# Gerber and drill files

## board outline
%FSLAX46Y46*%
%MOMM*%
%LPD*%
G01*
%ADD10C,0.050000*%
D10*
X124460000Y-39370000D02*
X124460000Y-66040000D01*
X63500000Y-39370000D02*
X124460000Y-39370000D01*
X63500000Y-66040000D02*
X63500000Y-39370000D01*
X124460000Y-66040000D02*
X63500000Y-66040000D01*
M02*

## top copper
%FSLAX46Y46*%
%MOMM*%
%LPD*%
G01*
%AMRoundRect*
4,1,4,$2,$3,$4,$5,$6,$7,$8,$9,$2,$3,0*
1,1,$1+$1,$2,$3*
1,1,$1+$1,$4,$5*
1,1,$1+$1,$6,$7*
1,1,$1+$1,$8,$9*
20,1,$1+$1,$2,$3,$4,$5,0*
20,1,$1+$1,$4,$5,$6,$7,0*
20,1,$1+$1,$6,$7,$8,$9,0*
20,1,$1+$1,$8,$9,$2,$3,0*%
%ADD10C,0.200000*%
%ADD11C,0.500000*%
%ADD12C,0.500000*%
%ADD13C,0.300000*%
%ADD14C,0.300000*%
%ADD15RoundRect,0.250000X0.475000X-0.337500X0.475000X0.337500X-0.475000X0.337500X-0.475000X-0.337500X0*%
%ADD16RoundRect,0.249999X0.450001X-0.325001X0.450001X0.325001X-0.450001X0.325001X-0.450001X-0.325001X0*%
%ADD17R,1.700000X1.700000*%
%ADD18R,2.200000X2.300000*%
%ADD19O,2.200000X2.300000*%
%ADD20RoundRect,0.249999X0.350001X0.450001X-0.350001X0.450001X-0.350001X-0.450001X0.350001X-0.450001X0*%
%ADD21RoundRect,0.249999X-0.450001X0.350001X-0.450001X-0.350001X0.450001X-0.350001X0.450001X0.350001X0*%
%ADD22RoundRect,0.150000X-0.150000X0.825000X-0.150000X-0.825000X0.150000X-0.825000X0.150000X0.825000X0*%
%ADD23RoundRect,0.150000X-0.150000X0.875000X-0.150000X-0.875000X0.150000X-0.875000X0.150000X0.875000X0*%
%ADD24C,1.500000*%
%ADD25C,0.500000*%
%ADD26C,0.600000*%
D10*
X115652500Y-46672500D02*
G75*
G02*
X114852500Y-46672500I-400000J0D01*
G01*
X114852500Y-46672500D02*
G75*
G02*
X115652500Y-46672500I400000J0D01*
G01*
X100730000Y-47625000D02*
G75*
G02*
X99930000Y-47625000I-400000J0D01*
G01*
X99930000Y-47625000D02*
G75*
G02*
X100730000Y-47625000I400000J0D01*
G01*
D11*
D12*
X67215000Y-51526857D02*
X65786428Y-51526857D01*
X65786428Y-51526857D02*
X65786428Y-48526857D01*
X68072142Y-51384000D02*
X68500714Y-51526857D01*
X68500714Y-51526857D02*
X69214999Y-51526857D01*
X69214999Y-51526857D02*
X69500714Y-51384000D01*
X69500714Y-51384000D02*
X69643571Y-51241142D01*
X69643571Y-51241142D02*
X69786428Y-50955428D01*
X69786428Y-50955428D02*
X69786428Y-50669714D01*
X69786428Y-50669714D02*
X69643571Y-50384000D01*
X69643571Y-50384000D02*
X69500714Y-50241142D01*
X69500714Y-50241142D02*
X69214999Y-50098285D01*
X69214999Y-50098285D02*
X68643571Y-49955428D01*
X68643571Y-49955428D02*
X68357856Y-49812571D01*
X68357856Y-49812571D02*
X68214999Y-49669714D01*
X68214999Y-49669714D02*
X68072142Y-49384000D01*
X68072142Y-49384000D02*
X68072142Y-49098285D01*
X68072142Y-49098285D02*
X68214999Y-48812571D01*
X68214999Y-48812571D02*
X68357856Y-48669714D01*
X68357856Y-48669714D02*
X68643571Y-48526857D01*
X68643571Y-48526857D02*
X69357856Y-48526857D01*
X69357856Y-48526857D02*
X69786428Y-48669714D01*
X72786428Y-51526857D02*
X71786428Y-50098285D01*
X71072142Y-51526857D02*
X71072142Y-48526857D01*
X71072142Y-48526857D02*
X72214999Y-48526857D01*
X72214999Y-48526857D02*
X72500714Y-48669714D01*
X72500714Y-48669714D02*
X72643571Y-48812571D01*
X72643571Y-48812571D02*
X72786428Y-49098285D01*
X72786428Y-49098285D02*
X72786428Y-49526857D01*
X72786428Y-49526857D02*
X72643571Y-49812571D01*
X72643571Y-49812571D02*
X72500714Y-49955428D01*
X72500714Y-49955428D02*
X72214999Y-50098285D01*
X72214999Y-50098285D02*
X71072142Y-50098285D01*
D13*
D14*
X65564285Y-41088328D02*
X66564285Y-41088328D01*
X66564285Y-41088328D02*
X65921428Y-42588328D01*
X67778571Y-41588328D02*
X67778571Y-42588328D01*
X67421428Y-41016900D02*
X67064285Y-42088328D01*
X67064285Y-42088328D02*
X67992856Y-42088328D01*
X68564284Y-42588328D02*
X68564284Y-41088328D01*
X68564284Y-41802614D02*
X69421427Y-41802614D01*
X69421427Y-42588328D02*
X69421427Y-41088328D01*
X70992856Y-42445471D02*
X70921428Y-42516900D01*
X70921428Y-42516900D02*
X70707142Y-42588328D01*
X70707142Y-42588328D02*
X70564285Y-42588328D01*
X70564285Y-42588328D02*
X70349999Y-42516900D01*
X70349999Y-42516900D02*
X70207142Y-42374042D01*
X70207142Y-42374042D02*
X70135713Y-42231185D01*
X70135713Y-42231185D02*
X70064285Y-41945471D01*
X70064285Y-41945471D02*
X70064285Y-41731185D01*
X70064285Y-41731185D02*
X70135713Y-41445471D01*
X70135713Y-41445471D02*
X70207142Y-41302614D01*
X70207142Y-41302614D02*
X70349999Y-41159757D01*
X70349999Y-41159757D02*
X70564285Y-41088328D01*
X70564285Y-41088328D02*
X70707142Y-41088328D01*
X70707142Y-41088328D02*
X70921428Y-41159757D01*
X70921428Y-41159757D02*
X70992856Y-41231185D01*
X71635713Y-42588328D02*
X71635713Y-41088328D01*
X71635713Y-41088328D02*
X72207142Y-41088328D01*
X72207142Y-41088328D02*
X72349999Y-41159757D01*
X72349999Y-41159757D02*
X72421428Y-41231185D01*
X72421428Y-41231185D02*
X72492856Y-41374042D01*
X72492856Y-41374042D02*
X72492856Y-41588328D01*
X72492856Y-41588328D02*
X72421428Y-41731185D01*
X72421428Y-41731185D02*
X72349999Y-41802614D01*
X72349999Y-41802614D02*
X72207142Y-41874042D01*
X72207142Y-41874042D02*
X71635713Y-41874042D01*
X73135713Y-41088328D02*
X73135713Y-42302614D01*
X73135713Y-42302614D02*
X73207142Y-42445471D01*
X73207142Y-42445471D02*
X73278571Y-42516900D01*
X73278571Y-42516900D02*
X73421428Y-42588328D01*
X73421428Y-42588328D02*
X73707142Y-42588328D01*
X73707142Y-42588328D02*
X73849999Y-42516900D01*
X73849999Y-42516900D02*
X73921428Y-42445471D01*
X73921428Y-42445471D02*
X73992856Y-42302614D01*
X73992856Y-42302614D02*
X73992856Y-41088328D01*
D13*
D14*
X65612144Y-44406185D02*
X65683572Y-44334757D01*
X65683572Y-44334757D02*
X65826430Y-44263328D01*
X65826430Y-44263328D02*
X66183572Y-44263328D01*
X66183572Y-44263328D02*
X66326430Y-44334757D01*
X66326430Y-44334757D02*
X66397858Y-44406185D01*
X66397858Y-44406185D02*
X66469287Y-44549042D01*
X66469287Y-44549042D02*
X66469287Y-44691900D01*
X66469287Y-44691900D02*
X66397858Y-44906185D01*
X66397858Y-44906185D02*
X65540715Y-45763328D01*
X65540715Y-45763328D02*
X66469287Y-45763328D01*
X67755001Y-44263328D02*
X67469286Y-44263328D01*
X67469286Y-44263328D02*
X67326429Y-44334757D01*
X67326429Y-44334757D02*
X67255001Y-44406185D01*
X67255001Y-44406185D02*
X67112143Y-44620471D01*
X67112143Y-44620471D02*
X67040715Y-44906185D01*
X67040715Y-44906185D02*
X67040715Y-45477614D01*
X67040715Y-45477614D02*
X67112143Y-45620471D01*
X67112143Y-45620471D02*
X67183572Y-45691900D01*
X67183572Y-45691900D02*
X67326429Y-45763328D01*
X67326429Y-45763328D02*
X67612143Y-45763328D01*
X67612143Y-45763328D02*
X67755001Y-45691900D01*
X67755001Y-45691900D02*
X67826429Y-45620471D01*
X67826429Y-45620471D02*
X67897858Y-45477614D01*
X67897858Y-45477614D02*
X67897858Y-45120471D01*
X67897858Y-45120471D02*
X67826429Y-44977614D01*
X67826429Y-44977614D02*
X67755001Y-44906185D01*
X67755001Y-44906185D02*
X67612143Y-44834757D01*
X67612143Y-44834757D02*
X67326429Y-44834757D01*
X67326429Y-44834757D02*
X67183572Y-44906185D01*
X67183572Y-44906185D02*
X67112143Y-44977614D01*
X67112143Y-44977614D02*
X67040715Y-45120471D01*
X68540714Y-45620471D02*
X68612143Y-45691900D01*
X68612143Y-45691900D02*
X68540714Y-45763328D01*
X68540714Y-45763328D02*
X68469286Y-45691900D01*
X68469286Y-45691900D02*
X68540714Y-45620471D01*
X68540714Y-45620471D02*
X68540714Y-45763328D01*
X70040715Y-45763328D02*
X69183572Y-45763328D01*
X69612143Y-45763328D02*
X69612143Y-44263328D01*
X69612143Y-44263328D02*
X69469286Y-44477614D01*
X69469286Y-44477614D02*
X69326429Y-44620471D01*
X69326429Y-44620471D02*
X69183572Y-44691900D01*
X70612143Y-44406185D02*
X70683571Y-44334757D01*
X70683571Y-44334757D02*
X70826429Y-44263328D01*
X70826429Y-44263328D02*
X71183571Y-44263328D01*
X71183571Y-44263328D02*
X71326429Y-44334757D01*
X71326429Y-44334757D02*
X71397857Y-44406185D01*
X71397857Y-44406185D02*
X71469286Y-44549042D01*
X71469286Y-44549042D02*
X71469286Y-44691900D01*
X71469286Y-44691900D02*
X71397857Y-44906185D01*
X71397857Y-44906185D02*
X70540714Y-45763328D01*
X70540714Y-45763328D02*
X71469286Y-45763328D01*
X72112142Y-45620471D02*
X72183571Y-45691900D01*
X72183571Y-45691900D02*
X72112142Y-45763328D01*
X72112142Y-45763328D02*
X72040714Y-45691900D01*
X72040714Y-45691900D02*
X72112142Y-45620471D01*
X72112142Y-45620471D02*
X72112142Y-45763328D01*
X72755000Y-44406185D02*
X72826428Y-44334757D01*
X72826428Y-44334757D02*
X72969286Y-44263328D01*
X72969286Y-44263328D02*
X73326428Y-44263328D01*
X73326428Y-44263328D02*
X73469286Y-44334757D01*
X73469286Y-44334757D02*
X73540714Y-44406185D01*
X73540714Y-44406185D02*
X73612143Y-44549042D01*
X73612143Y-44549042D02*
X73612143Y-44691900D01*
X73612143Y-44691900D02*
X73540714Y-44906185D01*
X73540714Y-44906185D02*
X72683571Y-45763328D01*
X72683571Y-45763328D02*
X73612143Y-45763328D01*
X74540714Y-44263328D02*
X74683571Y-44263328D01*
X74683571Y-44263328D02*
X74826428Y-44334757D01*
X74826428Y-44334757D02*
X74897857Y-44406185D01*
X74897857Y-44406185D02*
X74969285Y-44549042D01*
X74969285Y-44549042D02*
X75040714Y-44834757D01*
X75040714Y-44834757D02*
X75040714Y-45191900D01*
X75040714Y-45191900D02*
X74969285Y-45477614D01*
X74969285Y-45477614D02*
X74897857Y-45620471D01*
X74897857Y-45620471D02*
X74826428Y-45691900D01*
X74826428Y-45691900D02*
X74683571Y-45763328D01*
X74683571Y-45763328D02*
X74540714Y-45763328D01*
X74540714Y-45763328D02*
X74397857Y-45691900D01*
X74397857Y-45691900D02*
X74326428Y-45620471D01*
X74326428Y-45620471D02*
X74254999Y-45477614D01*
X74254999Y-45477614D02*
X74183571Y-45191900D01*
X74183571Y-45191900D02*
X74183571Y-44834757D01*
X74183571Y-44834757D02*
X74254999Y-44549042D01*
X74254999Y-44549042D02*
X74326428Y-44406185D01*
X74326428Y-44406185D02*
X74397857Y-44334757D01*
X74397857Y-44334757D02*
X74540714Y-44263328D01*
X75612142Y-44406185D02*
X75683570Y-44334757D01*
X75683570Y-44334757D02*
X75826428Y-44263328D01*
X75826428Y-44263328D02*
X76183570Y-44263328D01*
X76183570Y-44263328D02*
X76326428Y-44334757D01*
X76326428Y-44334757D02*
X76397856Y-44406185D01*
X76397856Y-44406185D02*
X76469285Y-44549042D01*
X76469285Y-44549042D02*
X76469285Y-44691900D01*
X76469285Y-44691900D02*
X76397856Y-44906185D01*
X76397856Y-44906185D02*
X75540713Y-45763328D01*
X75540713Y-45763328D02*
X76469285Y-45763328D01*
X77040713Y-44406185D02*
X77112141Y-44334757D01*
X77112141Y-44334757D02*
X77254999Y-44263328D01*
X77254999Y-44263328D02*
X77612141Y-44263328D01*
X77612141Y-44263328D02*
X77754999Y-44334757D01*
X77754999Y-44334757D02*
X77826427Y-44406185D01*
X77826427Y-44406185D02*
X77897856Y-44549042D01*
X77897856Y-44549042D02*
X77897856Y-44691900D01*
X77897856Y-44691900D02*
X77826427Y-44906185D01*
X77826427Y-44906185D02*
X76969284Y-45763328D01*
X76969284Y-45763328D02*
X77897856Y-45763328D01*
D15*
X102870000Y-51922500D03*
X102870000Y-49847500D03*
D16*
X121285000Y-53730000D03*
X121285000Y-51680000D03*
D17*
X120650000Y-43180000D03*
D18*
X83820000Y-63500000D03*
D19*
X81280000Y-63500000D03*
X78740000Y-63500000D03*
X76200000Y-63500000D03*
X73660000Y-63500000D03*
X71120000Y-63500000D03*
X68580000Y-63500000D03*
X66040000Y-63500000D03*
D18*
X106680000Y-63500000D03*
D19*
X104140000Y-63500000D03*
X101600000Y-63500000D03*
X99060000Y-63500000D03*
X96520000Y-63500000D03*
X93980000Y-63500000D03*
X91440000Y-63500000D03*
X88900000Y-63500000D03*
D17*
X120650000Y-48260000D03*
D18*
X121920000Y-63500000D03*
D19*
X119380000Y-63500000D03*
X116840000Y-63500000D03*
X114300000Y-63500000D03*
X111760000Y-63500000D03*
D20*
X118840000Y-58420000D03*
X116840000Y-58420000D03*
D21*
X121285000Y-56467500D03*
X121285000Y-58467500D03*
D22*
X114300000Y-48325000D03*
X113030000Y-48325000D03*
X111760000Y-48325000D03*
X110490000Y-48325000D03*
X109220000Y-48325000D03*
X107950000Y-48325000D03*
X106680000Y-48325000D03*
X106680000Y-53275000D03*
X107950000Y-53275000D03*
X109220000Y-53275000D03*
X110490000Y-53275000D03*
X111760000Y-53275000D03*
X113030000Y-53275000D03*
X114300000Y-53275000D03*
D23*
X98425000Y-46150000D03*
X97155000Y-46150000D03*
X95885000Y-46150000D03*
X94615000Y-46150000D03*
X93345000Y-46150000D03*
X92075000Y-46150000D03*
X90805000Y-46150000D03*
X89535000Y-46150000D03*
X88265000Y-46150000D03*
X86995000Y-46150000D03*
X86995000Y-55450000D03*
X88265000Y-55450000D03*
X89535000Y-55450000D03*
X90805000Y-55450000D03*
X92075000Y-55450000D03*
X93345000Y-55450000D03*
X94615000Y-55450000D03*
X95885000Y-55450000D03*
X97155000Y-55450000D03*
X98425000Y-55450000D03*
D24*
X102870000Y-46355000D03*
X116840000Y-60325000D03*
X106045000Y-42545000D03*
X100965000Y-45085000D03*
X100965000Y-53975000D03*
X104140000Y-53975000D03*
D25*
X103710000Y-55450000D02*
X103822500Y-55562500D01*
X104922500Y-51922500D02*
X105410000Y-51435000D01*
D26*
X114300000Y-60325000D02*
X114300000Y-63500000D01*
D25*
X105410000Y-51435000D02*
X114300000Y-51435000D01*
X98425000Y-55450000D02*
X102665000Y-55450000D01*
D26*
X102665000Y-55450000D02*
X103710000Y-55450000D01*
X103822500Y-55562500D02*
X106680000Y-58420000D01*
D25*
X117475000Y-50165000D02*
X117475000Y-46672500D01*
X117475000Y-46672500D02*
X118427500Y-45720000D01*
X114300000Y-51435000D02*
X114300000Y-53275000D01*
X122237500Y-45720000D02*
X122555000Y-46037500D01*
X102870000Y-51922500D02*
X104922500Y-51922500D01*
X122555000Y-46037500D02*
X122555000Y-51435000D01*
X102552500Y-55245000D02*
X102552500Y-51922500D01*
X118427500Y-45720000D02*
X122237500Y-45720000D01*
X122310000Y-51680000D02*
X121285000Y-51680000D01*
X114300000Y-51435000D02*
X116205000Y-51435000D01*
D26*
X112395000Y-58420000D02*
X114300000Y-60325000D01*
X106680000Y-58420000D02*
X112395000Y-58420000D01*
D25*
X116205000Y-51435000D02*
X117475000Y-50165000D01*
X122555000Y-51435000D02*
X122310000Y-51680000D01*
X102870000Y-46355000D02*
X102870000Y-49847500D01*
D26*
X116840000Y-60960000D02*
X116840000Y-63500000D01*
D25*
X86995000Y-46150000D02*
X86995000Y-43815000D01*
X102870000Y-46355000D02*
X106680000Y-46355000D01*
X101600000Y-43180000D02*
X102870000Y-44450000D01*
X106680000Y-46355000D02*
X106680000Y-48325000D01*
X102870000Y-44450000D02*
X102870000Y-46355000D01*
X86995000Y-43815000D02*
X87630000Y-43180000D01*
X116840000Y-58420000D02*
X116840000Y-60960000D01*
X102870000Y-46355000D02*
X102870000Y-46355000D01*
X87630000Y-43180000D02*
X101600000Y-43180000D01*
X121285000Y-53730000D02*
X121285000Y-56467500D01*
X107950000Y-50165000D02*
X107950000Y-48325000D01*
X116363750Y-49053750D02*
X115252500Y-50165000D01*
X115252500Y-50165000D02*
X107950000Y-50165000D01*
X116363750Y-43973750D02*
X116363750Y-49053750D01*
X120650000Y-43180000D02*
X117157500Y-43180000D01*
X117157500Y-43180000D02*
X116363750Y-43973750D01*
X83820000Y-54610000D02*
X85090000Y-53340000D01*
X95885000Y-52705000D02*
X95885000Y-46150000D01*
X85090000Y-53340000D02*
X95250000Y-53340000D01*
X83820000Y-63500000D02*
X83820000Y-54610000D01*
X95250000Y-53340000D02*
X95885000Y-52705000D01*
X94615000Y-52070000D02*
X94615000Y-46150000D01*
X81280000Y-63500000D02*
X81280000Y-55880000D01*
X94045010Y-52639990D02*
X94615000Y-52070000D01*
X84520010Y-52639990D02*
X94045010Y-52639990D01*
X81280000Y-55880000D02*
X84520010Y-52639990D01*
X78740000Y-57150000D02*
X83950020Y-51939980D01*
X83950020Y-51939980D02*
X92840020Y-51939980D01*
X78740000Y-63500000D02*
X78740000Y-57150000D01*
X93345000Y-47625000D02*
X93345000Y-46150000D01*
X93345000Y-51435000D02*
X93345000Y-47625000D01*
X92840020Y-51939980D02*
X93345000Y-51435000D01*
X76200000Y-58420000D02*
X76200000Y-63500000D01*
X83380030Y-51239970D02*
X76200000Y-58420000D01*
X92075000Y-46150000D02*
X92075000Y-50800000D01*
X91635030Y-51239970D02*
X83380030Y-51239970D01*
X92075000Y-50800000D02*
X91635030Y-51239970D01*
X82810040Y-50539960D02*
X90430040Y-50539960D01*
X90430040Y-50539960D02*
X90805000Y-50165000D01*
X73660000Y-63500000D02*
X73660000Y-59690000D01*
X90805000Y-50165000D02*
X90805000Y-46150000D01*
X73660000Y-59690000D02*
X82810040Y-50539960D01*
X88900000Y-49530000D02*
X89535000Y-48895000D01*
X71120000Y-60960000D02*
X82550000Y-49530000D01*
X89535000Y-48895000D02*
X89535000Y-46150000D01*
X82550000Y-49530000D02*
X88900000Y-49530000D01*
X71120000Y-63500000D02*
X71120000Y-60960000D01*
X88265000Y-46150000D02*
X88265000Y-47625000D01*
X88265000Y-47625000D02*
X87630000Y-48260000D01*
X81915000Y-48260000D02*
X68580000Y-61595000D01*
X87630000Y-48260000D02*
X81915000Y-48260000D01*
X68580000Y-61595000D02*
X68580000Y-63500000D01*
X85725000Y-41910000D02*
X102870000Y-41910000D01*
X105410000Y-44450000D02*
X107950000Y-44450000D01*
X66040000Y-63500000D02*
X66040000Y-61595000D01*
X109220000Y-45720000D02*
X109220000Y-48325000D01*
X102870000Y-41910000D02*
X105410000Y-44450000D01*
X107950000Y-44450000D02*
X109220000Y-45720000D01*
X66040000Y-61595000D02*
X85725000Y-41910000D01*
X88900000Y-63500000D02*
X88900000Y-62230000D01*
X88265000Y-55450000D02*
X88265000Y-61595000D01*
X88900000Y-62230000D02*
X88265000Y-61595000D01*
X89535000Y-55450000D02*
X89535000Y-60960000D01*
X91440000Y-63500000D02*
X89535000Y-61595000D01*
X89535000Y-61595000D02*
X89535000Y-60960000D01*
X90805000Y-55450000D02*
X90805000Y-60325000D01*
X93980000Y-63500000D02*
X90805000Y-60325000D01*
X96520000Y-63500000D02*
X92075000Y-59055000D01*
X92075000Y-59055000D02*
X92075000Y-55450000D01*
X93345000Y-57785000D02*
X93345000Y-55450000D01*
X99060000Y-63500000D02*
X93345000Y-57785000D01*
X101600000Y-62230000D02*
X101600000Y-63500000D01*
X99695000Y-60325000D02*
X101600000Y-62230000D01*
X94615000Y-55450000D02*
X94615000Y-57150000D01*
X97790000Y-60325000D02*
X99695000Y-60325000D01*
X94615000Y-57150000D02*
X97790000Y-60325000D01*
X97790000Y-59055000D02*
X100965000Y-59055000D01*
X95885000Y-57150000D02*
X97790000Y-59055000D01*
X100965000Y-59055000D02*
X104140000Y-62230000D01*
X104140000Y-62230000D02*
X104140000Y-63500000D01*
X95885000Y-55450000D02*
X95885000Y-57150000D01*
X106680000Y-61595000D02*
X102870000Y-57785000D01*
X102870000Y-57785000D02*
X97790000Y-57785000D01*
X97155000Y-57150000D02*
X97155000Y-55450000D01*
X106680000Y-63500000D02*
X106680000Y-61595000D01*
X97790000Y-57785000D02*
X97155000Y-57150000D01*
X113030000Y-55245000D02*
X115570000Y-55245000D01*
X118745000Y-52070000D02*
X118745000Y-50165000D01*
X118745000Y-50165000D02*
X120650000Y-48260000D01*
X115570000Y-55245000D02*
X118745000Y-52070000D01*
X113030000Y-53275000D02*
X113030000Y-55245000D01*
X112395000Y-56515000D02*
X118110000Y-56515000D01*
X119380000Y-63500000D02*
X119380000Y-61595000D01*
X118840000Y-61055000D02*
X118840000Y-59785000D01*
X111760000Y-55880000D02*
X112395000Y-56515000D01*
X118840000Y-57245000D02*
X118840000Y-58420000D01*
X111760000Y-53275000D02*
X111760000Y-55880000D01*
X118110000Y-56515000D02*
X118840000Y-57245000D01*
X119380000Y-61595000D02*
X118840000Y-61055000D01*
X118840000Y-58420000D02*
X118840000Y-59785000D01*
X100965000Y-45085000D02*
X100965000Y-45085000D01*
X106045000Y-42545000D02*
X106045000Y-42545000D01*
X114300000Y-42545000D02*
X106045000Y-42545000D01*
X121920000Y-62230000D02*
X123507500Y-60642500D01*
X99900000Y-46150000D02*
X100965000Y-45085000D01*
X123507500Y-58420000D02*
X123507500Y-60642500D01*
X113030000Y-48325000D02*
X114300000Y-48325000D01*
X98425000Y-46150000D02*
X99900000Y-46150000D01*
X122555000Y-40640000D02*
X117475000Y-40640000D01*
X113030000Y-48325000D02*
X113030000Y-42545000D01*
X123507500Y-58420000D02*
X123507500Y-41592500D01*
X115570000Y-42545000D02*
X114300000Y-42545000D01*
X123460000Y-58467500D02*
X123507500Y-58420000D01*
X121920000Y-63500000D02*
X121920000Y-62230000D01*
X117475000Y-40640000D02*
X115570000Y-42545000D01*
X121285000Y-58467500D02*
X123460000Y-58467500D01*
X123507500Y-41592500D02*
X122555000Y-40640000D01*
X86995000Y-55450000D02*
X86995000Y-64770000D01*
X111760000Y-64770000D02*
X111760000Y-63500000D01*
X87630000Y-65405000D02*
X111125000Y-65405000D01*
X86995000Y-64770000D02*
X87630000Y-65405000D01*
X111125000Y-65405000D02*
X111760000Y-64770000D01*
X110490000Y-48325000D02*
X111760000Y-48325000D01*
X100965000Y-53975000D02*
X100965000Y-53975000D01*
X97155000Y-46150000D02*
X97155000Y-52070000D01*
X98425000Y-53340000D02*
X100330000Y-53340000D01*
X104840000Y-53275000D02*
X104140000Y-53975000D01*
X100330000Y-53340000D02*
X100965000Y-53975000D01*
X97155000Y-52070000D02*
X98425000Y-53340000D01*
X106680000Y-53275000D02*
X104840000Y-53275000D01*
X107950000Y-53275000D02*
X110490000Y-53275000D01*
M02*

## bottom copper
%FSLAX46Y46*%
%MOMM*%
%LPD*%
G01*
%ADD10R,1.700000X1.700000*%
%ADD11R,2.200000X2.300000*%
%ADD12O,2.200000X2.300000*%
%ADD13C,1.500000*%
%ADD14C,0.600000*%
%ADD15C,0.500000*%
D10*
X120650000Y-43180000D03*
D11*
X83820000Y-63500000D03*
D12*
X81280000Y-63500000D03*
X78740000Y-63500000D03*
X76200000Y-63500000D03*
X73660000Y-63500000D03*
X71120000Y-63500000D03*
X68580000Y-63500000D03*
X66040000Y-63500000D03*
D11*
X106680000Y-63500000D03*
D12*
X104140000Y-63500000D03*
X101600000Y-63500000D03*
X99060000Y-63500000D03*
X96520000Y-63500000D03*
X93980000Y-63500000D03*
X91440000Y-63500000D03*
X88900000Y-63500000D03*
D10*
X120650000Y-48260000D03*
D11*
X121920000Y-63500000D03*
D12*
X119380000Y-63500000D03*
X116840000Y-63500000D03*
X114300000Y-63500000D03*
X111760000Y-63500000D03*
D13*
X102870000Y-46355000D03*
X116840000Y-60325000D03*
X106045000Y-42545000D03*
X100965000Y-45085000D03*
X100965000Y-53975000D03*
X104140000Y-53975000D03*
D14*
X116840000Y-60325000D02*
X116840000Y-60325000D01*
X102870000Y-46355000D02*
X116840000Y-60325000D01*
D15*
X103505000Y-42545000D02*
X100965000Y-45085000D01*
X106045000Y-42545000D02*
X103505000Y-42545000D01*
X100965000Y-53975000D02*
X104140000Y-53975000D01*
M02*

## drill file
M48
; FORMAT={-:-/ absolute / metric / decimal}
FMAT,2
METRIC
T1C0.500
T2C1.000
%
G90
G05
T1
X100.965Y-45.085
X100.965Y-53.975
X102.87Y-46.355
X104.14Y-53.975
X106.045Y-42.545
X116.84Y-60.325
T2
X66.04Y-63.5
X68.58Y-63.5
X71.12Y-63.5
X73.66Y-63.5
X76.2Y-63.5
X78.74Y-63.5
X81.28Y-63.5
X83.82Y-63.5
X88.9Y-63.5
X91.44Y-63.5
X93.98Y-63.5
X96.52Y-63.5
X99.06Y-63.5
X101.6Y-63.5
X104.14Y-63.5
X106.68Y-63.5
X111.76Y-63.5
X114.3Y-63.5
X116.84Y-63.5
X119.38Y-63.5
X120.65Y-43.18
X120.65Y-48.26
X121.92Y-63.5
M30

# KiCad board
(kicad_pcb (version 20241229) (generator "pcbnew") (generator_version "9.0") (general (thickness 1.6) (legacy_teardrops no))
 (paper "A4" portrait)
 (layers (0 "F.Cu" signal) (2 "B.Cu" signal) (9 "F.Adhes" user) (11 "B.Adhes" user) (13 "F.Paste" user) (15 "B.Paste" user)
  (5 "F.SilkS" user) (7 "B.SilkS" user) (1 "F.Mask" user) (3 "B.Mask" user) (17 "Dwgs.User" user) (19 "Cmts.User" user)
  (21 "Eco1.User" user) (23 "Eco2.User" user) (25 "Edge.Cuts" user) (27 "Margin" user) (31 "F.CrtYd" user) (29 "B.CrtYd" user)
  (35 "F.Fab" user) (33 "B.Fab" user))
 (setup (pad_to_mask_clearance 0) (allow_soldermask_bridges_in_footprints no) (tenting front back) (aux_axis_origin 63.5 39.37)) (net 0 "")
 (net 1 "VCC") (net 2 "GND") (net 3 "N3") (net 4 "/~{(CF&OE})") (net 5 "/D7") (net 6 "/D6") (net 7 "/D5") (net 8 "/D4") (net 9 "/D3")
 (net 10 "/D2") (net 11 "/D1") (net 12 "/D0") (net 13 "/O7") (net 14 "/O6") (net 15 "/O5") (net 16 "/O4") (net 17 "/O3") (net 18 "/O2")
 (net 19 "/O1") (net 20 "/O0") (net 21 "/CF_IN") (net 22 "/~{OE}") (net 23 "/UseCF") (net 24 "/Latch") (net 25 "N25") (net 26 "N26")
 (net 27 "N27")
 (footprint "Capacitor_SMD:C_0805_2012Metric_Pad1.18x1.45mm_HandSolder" (layer "F.Cu") (at 102.87 50.885 90)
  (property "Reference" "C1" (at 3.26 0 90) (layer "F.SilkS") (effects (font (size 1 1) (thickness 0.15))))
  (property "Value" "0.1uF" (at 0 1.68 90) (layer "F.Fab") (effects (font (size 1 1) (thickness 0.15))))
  (pad "1" smd roundrect (at -1.0375 0 90) (size 1.175 1.45) (layers "F.Cu" "F.Mask" "F.Paste") (roundrect_rratio 0.2127659574)
   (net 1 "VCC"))
  (pad "2" smd roundrect (at 1.0375 0 90) (size 1.175 1.45) (layers "F.Cu" "F.Mask" "F.Paste") (roundrect_rratio 0.2127659574) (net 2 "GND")))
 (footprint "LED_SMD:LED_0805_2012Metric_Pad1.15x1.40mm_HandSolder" (layer "F.Cu") (at 121.285 52.705 90)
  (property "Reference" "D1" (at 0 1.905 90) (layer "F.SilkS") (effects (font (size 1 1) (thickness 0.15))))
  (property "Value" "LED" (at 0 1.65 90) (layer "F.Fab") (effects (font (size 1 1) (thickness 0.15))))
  (pad "1" smd roundrect (at -1.025 0 90) (size 1.15 1.4) (layers "F.Cu" "F.Mask" "F.Paste") (roundrect_rratio 0.2173904348) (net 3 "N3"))
  (pad "2" smd roundrect (at 1.025 0 90) (size 1.15 1.4) (layers "F.Cu" "F.Mask" "F.Paste") (roundrect_rratio 0.2173904348) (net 1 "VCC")))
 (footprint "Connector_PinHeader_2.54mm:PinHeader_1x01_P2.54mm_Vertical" (layer "F.Cu") (at 120.65 43.18)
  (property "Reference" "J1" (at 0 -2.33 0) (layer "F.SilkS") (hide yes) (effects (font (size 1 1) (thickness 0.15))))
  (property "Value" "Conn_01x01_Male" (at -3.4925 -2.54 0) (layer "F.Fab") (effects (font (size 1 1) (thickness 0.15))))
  (pad "1" thru_hole rect (at 0 0) (size 1.7 1.7) (drill 1) (layers "*.Cu" "*.Mask") (remove_unused_layers no) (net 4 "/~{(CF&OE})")))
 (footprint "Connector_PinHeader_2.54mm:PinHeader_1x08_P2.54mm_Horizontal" (layer "F.Cu") (at 83.82 63.5 -90)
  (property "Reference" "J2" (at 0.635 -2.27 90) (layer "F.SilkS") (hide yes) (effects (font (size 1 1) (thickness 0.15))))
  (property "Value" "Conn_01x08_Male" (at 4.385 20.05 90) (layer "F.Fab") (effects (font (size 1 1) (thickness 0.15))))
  (pad "1" thru_hole rect (at 0 0 270) (size 2.3 2.2) (drill 1) (layers "*.Cu" "*.Mask") (remove_unused_layers no) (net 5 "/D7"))
  (pad "2" thru_hole oval (at 0 2.54 270) (size 2.3 2.2) (drill 1) (layers "*.Cu" "*.Mask") (remove_unused_layers no) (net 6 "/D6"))
  (pad "3" thru_hole oval (at 0 5.08 270) (size 2.3 2.2) (drill 1) (layers "*.Cu" "*.Mask") (remove_unused_layers no) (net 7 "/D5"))
  (pad "4" thru_hole oval (at 0 7.62 270) (size 2.3 2.2) (drill 1) (layers "*.Cu" "*.Mask") (remove_unused_layers no) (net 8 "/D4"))
  (pad "5" thru_hole oval (at 0 10.16 270) (size 2.3 2.2) (drill 1) (layers "*.Cu" "*.Mask") (remove_unused_layers no) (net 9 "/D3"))
  (pad "6" thru_hole oval (at 0 12.7 270) (size 2.3 2.2) (drill 1) (layers "*.Cu" "*.Mask") (remove_unused_layers no) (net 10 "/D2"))
  (pad "7" thru_hole oval (at 0 15.24 270) (size 2.3 2.2) (drill 1) (layers "*.Cu" "*.Mask") (remove_unused_layers no) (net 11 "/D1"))
  (pad "8" thru_hole oval (at 0 17.78 270) (size 2.3 2.2) (drill 1) (layers "*.Cu" "*.Mask") (remove_unused_layers no) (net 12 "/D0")))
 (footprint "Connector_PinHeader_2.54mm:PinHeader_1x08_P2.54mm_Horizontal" (layer "F.Cu") (at 106.68 63.5 -90)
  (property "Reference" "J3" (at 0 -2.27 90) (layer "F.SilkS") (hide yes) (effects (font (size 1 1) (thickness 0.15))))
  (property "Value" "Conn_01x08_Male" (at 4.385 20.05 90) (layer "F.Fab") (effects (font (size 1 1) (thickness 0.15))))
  (pad "1" thru_hole rect (at 0 0 270) (size 2.3 2.2) (drill 1) (layers "*.Cu" "*.Mask") (remove_unused_layers no) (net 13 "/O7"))
  (pad "2" thru_hole oval (at 0 2.54 270) (size 2.3 2.2) (drill 1) (layers "*.Cu" "*.Mask") (remove_unused_layers no) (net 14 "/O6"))
  (pad "3" thru_hole oval (at 0 5.08 270) (size 2.3 2.2) (drill 1) (layers "*.Cu" "*.Mask") (remove_unused_layers no) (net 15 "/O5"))
  (pad "4" thru_hole oval (at 0 7.62 270) (size 2.3 2.2) (drill 1) (layers "*.Cu" "*.Mask") (remove_unused_layers no) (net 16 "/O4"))
  (pad "5" thru_hole oval (at 0 10.16 270) (size 2.3 2.2) (drill 1) (layers "*.Cu" "*.Mask") (remove_unused_layers no) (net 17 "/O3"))
  (pad "6" thru_hole oval (at 0 12.7 270) (size 2.3 2.2) (drill 1) (layers "*.Cu" "*.Mask") (remove_unused_layers no) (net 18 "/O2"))
  (pad "7" thru_hole oval (at 0 15.24 270) (size 2.3 2.2) (drill 1) (layers "*.Cu" "*.Mask") (remove_unused_layers no) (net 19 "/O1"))
  (pad "8" thru_hole oval (at 0 17.78 270) (size 2.3 2.2) (drill 1) (layers "*.Cu" "*.Mask") (remove_unused_layers no) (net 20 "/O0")))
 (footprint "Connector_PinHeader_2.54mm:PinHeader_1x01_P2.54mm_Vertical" (layer "F.Cu") (at 120.65 48.26)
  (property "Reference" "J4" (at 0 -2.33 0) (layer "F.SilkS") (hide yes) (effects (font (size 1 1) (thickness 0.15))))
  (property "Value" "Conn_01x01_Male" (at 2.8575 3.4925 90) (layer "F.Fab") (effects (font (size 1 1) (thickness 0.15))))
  (pad "1" thru_hole rect (at 0 0) (size 1.7 1.7) (drill 1) (layers "*.Cu" "*.Mask") (remove_unused_layers no) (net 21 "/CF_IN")))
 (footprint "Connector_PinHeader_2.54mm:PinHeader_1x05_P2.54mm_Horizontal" (layer "F.Cu") (at 121.92 63.5 -90)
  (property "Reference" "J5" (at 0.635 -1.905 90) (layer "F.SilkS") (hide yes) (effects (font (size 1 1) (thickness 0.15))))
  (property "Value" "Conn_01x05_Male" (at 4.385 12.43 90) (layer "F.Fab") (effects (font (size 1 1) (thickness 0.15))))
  (pad "1" thru_hole rect (at 0 0 270) (size 2.3 2.2) (drill 1) (layers "*.Cu" "*.Mask") (remove_unused_layers no) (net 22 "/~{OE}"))
  (pad "2" thru_hole oval (at 0 2.54 270) (size 2.3 2.2) (drill 1) (layers "*.Cu" "*.Mask") (remove_unused_layers no) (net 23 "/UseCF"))
  (pad "3" thru_hole oval (at 0 5.08 270) (size 2.3 2.2) (drill 1) (layers "*.Cu" "*.Mask") (remove_unused_layers no) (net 2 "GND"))
  (pad "4" thru_hole oval (at 0 7.62 270) (size 2.3 2.2) (drill 1) (layers "*.Cu" "*.Mask") (remove_unused_layers no) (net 1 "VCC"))
  (pad "5" thru_hole oval (at 0 10.16 270) (size 2.3 2.2) (drill 1) (layers "*.Cu" "*.Mask") (remove_unused_layers no) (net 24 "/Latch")))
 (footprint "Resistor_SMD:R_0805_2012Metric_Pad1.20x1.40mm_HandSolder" (layer "F.Cu") (at 117.84 58.42 180)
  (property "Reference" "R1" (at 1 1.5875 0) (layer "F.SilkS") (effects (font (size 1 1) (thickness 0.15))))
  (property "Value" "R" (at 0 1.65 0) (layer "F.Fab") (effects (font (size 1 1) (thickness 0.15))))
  (pad "1" smd roundrect (at -1 0 180) (size 1.2 1.4) (layers "F.Cu" "F.Mask" "F.Paste") (roundrect_rratio 0.2083325) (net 23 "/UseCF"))
  (pad "2" smd roundrect (at 1 0 180) (size 1.2 1.4) (layers "F.Cu" "F.Mask" "F.Paste") (roundrect_rratio 0.2083325) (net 2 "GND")))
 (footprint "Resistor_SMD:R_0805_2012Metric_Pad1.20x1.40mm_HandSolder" (layer "F.Cu") (at 121.285 57.4675 -90)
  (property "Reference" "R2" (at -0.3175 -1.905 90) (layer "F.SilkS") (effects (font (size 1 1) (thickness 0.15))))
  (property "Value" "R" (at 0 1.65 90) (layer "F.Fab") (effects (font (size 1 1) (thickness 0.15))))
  (pad "1" smd roundrect (at -1 0 270) (size 1.2 1.4) (layers "F.Cu" "F.Mask" "F.Paste") (roundrect_rratio 0.2083325) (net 3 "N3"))
  (pad "2" smd roundrect (at 1 0 270) (size 1.2 1.4) (layers "F.Cu" "F.Mask" "F.Paste") (roundrect_rratio 0.2083325) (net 22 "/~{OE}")))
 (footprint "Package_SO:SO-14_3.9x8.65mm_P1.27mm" (layer "F.Cu") (at 110.49 50.8 -90)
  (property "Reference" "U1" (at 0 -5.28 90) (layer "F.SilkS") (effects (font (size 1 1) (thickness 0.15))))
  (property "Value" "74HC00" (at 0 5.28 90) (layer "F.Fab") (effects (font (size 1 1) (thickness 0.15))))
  (pad "1" smd roundrect (at -2.475 -3.81 270) (size 1.95 0.6) (layers "F.Cu" "F.Mask" "F.Paste") (roundrect_rratio 0.25) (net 22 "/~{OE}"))
  (pad "2" smd roundrect (at -2.475 -2.54 270) (size 1.95 0.6) (layers "F.Cu" "F.Mask" "F.Paste") (roundrect_rratio 0.25) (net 22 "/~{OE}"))
  (pad "3" smd roundrect (at -2.475 -1.27 270) (size 1.95 0.6) (layers "F.Cu" "F.Mask" "F.Paste") (roundrect_rratio 0.25) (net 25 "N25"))
  (pad "4" smd roundrect (at -2.475 0 270) (size 1.95 0.6) (layers "F.Cu" "F.Mask" "F.Paste") (roundrect_rratio 0.25) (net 25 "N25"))
  (pad "5" smd roundrect (at -2.475 1.27 270) (size 1.95 0.6) (layers "F.Cu" "F.Mask" "F.Paste") (roundrect_rratio 0.25) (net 12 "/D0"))
  (pad "6" smd roundrect (at -2.475 2.54 270) (size 1.95 0.6) (layers "F.Cu" "F.Mask" "F.Paste") (roundrect_rratio 0.25)
   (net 4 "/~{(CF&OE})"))
  (pad "7" smd roundrect (at -2.475 3.81 270) (size 1.95 0.6) (layers "F.Cu" "F.Mask" "F.Paste") (roundrect_rratio 0.25) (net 2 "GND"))
  (pad "8" smd roundrect (at 2.475 3.81 270) (size 1.95 0.6) (layers "F.Cu" "F.Mask" "F.Paste") (roundrect_rratio 0.25) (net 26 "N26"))
  (pad "9" smd roundrect (at 2.475 2.54 270) (size 1.95 0.6) (layers "F.Cu" "F.Mask" "F.Paste") (roundrect_rratio 0.25) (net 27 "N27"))
  (pad "10" smd roundrect (at 2.475 1.27 270) (size 1.95 0.6) (layers "F.Cu" "F.Mask" "F.Paste") (roundrect_rratio 0.25) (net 27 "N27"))
  (pad "11" smd roundrect (at 2.475 0 270) (size 1.95 0.6) (layers "F.Cu" "F.Mask" "F.Paste") (roundrect_rratio 0.25) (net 27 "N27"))
  (pad "12" smd roundrect (at 2.475 -1.27 270) (size 1.95 0.6) (layers "F.Cu" "F.Mask" "F.Paste") (roundrect_rratio 0.25) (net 23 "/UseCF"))
  (pad "13" smd roundrect (at 2.475 -2.54 270) (size 1.95 0.6) (layers "F.Cu" "F.Mask" "F.Paste") (roundrect_rratio 0.25) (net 21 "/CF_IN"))
  (pad "14" smd roundrect (at 2.475 -3.81 270) (size 1.95 0.6) (layers "F.Cu" "F.Mask" "F.Paste") (roundrect_rratio 0.25) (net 1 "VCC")))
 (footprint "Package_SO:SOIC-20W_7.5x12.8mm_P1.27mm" (layer "F.Cu") (at 92.71 50.8 -90)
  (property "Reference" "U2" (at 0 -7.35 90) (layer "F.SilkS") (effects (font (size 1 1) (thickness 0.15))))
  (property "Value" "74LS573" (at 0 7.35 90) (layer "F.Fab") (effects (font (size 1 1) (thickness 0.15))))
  (pad "1" smd roundrect (at -4.65 -5.715 270) (size 2.05 0.6) (layers "F.Cu" "F.Mask" "F.Paste") (roundrect_rratio 0.25) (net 22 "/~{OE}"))
  (pad "2" smd roundrect (at -4.65 -4.445 270) (size 2.05 0.6) (layers "F.Cu" "F.Mask" "F.Paste") (roundrect_rratio 0.25) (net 26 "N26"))
  (pad "3" smd roundrect (at -4.65 -3.175 270) (size 2.05 0.6) (layers "F.Cu" "F.Mask" "F.Paste") (roundrect_rratio 0.25) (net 5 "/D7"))
  (pad "4" smd roundrect (at -4.65 -1.905 270) (size 2.05 0.6) (layers "F.Cu" "F.Mask" "F.Paste") (roundrect_rratio 0.25) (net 6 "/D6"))
  (pad "5" smd roundrect (at -4.65 -0.635 270) (size 2.05 0.6) (layers "F.Cu" "F.Mask" "F.Paste") (roundrect_rratio 0.25) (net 7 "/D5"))
  (pad "6" smd roundrect (at -4.65 0.635 270) (size 2.05 0.6) (layers "F.Cu" "F.Mask" "F.Paste") (roundrect_rratio 0.25) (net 8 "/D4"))
  (pad "7" smd roundrect (at -4.65 1.905 270) (size 2.05 0.6) (layers "F.Cu" "F.Mask" "F.Paste") (roundrect_rratio 0.25) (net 9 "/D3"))
  (pad "8" smd roundrect (at -4.65 3.175 270) (size 2.05 0.6) (layers "F.Cu" "F.Mask" "F.Paste") (roundrect_rratio 0.25) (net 10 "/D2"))
  (pad "9" smd roundrect (at -4.65 4.445 270) (size 2.05 0.6) (layers "F.Cu" "F.Mask" "F.Paste") (roundrect_rratio 0.25) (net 11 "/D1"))
  (pad "10" smd roundrect (at -4.65 5.715 270) (size 2.05 0.6) (layers "F.Cu" "F.Mask" "F.Paste") (roundrect_rratio 0.25) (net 2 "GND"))
  (pad "11" smd roundrect (at 4.65 5.715 270) (size 2.05 0.6) (layers "F.Cu" "F.Mask" "F.Paste") (roundrect_rratio 0.25) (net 24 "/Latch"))
  (pad "12" smd roundrect (at 4.65 4.445 270) (size 2.05 0.6) (layers "F.Cu" "F.Mask" "F.Paste") (roundrect_rratio 0.25) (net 20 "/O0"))
  (pad "13" smd roundrect (at 4.65 3.175 270) (size 2.05 0.6) (layers "F.Cu" "F.Mask" "F.Paste") (roundrect_rratio 0.25) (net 19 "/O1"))
  (pad "14" smd roundrect (at 4.65 1.905 270) (size 2.05 0.6) (layers "F.Cu" "F.Mask" "F.Paste") (roundrect_rratio 0.25) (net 18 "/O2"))
  (pad "15" smd roundrect (at 4.65 0.635 270) (size 2.05 0.6) (layers "F.Cu" "F.Mask" "F.Paste") (roundrect_rratio 0.25) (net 17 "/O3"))
  (pad "16" smd roundrect (at 4.65 -0.635 270) (size 2.05 0.6) (layers "F.Cu" "F.Mask" "F.Paste") (roundrect_rratio 0.25) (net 16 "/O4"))
  (pad "17" smd roundrect (at 4.65 -1.905 270) (size 2.05 0.6) (layers "F.Cu" "F.Mask" "F.Paste") (roundrect_rratio 0.25) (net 15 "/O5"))
  (pad "18" smd roundrect (at 4.65 -3.175 270) (size 2.05 0.6) (layers "F.Cu" "F.Mask" "F.Paste") (roundrect_rratio 0.25) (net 14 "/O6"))
  (pad "19" smd roundrect (at 4.65 -4.445 270) (size 2.05 0.6) (layers "F.Cu" "F.Mask" "F.Paste") (roundrect_rratio 0.25) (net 13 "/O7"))
  (pad "20" smd roundrect (at 4.65 -5.715 270) (size 2.05 0.6) (layers "F.Cu" "F.Mask" "F.Paste") (roundrect_rratio 0.25) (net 1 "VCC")))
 (gr_circle (center 115.2525 46.6725) (end 115.6525 46.6725) (stroke (width 0.2) (type solid)) (fill no) (layer "F.Cu"))
 (gr_circle (center 100.33 47.625) (end 100.73 47.625) (stroke (width 0.2) (type solid)) (fill no) (layer "F.Cu"))
 (gr_line (start 124.46 39.37) (end 124.46 66.04) (stroke (width 0.05) (type solid)) (layer "Edge.Cuts"))
 (gr_line (start 63.5 39.37) (end 124.46 39.37) (stroke (width 0.05) (type solid)) (layer "Edge.Cuts"))
 (gr_line (start 63.5 66.04) (end 63.5 39.37) (stroke (width 0.05) (type solid)) (layer "Edge.Cuts"))
 (gr_line (start 124.46 66.04) (end 63.5 66.04) (stroke (width 0.05) (type solid)) (layer "Edge.Cuts"))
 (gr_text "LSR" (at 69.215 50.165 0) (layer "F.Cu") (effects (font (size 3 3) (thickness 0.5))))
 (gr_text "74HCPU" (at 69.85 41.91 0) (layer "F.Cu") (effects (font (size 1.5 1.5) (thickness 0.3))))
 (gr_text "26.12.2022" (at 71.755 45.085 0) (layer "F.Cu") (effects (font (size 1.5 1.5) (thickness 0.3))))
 (segment (start 103.71 55.45) (end 103.8225 55.5625) (width 0.5) (layer "F.Cu") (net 1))
 (segment (start 104.9225 51.9225) (end 105.41 51.435) (width 0.5) (layer "F.Cu") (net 1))
 (segment (start 114.3 60.325) (end 114.3 63.5) (width 0.6) (layer "F.Cu") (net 1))
 (segment (start 105.41 51.435) (end 114.3 51.435) (width 0.5) (layer "F.Cu") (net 1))
 (segment (start 98.425 55.45) (end 102.665 55.45) (width 0.5) (layer "F.Cu") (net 1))
 (segment (start 102.665 55.45) (end 103.71 55.45) (width 0.6) (layer "F.Cu") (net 1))
 (segment (start 103.8225 55.5625) (end 106.68 58.42) (width 0.6) (layer "F.Cu") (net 1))
 (segment (start 117.475 50.165) (end 117.475 46.6725) (width 0.5) (layer "F.Cu") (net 1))
 (segment (start 117.475 46.6725) (end 118.4275 45.72) (width 0.5) (layer "F.Cu") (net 1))
 (segment (start 114.3 51.435) (end 114.3 53.275) (width 0.5) (layer "F.Cu") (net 1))
 (segment (start 122.2375 45.72) (end 122.555 46.0375) (width 0.5) (layer "F.Cu") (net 1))
 (segment (start 102.87 51.9225) (end 104.9225 51.9225) (width 0.5) (layer "F.Cu") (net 1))
 (segment (start 122.555 46.0375) (end 122.555 51.435) (width 0.5) (layer "F.Cu") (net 1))
 (segment (start 102.5525 55.245) (end 102.5525 51.9225) (width 0.5) (layer "F.Cu") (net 1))
 (segment (start 118.4275 45.72) (end 122.2375 45.72) (width 0.5) (layer "F.Cu") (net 1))
 (segment (start 122.31 51.68) (end 121.285 51.68) (width 0.5) (layer "F.Cu") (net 1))
 (segment (start 114.3 51.435) (end 116.205 51.435) (width 0.5) (layer "F.Cu") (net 1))
 (segment (start 112.395 58.42) (end 114.3 60.325) (width 0.6) (layer "F.Cu") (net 1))
 (segment (start 106.68 58.42) (end 112.395 58.42) (width 0.6) (layer "F.Cu") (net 1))
 (segment (start 116.205 51.435) (end 117.475 50.165) (width 0.5) (layer "F.Cu") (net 1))
 (segment (start 122.555 51.435) (end 122.31 51.68) (width 0.5) (layer "F.Cu") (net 1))
 (segment (start 102.87 46.355) (end 102.87 49.8475) (width 0.5) (layer "F.Cu") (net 2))
 (segment (start 116.84 60.96) (end 116.84 63.5) (width 0.6) (layer "F.Cu") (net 2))
 (segment (start 86.995 46.15) (end 86.995 43.815) (width 0.5) (layer "F.Cu") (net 2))
 (segment (start 102.87 46.355) (end 106.68 46.355) (width 0.5) (layer "F.Cu") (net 2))
 (segment (start 101.6 43.18) (end 102.87 44.45) (width 0.5) (layer "F.Cu") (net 2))
 (segment (start 106.68 46.355) (end 106.68 48.325) (width 0.5) (layer "F.Cu") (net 2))
 (segment (start 102.87 44.45) (end 102.87 46.355) (width 0.5) (layer "F.Cu") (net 2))
 (segment (start 86.995 43.815) (end 87.63 43.18) (width 0.5) (layer "F.Cu") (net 2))
 (segment (start 116.84 58.42) (end 116.84 60.96) (width 0.5) (layer "F.Cu") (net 2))
 (segment (start 102.87 46.355) (end 102.87 46.355) (width 0.5) (layer "F.Cu") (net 2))
 (segment (start 87.63 43.18) (end 101.6 43.18) (width 0.5) (layer "F.Cu") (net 2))
 (via (at 102.87 46.355) (size 1.5) (drill 0.5) (layers "F.Cu" "B.Cu") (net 2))
 (via (at 116.84 60.325) (size 1.5) (drill 0.5) (layers "F.Cu" "B.Cu") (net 2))
 (segment (start 116.84 60.325) (end 116.84 60.325) (width 0.6) (layer "B.Cu") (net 2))
 (segment (start 102.87 46.355) (end 116.84 60.325) (width 0.6) (layer "B.Cu") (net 2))
 (segment (start 121.285 53.73) (end 121.285 56.4675) (width 0.5) (layer "F.Cu") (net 3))
 (segment (start 107.95 50.165) (end 107.95 48.325) (width 0.5) (layer "F.Cu") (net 4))
 (segment (start 116.36375 49.05375) (end 115.2525 50.165) (width 0.5) (layer "F.Cu") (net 4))
 (segment (start 115.2525 50.165) (end 107.95 50.165) (width 0.5) (layer "F.Cu") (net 4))
 (segment (start 116.36375 43.97375) (end 116.36375 49.05375) (width 0.5) (layer "F.Cu") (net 4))
 (segment (start 120.65 43.18) (end 117.1575 43.18) (width 0.5) (layer "F.Cu") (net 4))
 (segment (start 117.1575 43.18) (end 116.36375 43.97375) (width 0.5) (layer "F.Cu") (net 4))
 (segment (start 83.82 54.61) (end 85.09 53.34) (width 0.5) (layer "F.Cu") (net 5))
 (segment (start 95.885 52.705) (end 95.885 46.15) (width 0.5) (layer "F.Cu") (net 5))
 (segment (start 85.09 53.34) (end 95.25 53.34) (width 0.5) (layer "F.Cu") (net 5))
 (segment (start 83.82 63.5) (end 83.82 54.61) (width 0.5) (layer "F.Cu") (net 5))
 (segment (start 95.25 53.34) (end 95.885 52.705) (width 0.5) (layer "F.Cu") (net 5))
 (segment (start 94.615 52.07) (end 94.615 46.15) (width 0.5) (layer "F.Cu") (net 6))
 (segment (start 81.28 63.5) (end 81.28 55.88) (width 0.5) (layer "F.Cu") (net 6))
 (segment (start 94.04501 52.63999) (end 94.615 52.07) (width 0.5) (layer "F.Cu") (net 6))
 (segment (start 84.52001 52.63999) (end 94.04501 52.63999) (width 0.5) (layer "F.Cu") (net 6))
 (segment (start 81.28 55.88) (end 84.52001 52.63999) (width 0.5) (layer "F.Cu") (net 6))
 (segment (start 78.74 57.15) (end 83.95002 51.93998) (width 0.5) (layer "F.Cu") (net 7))
 (segment (start 83.95002 51.93998) (end 92.84002 51.93998) (width 0.5) (layer "F.Cu") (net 7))
 (segment (start 78.74 63.5) (end 78.74 57.15) (width 0.5) (layer "F.Cu") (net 7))
 (segment (start 93.345 47.625) (end 93.345 46.15) (width 0.5) (layer "F.Cu") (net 7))
 (segment (start 93.345 51.435) (end 93.345 47.625) (width 0.5) (layer "F.Cu") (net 7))
 (segment (start 92.84002 51.93998) (end 93.345 51.435) (width 0.5) (layer "F.Cu") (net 7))
 (segment (start 76.2 58.42) (end 76.2 63.5) (width 0.5) (layer "F.Cu") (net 8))
 (segment (start 83.38003 51.23997) (end 76.2 58.42) (width 0.5) (layer "F.Cu") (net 8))
 (segment (start 92.075 46.15) (end 92.075 50.8) (width 0.5) (layer "F.Cu") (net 8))
 (segment (start 91.63503 51.23997) (end 83.38003 51.23997) (width 0.5) (layer "F.Cu") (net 8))
 (segment (start 92.075 50.8) (end 91.63503 51.23997) (width 0.5) (layer "F.Cu") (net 8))
 (segment (start 82.81004 50.53996) (end 90.43004 50.53996) (width 0.5) (layer "F.Cu") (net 9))
 (segment (start 90.43004 50.53996) (end 90.805 50.165) (width 0.5) (layer "F.Cu") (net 9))
 (segment (start 73.66 63.5) (end 73.66 59.69) (width 0.5) (layer "F.Cu") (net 9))
 (segment (start 90.805 50.165) (end 90.805 46.15) (width 0.5) (layer "F.Cu") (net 9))
 (segment (start 73.66 59.69) (end 82.81004 50.53996) (width 0.5) (layer "F.Cu") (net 9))
 (segment (start 88.9 49.53) (end 89.535 48.895) (width 0.5) (layer "F.Cu") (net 10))
 (segment (start 71.12 60.96) (end 82.55 49.53) (width 0.5) (layer "F.Cu") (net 10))
 (segment (start 89.535 48.895) (end 89.535 46.15) (width 0.5) (layer "F.Cu") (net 10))
 (segment (start 82.55 49.53) (end 88.9 49.53) (width 0.5) (layer "F.Cu") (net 10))
 (segment (start 71.12 63.5) (end 71.12 60.96) (width 0.5) (layer "F.Cu") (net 10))
 (segment (start 88.265 46.15) (end 88.265 47.625) (width 0.5) (layer "F.Cu") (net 11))
 (segment (start 88.265 47.625) (end 87.63 48.26) (width 0.5) (layer "F.Cu") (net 11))
 (segment (start 81.915 48.26) (end 68.58 61.595) (width 0.5) (layer "F.Cu") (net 11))
 (segment (start 87.63 48.26) (end 81.915 48.26) (width 0.5) (layer "F.Cu") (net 11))
 (segment (start 68.58 61.595) (end 68.58 63.5) (width 0.5) (layer "F.Cu") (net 11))
 (segment (start 85.725 41.91) (end 102.87 41.91) (width 0.5) (layer "F.Cu") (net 12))
 (segment (start 105.41 44.45) (end 107.95 44.45) (width 0.5) (layer "F.Cu") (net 12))
 (segment (start 66.04 63.5) (end 66.04 61.595) (width 0.5) (layer "F.Cu") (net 12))
 (segment (start 109.22 45.72) (end 109.22 48.325) (width 0.5) (layer "F.Cu") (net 12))
 (segment (start 102.87 41.91) (end 105.41 44.45) (width 0.5) (layer "F.Cu") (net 12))
 (segment (start 107.95 44.45) (end 109.22 45.72) (width 0.5) (layer "F.Cu") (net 12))
 (segment (start 66.04 61.595) (end 85.725 41.91) (width 0.5) (layer "F.Cu") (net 12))
 (segment (start 88.9 63.5) (end 88.9 62.23) (width 0.5) (layer "F.Cu") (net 20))
 (segment (start 88.265 55.45) (end 88.265 61.595) (width 0.5) (layer "F.Cu") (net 20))
 (segment (start 88.9 62.23) (end 88.265 61.595) (width 0.5) (layer "F.Cu") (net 20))
 (segment (start 89.535 55.45) (end 89.535 60.96) (width 0.5) (layer "F.Cu") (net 19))
 (segment (start 91.44 63.5) (end 89.535 61.595) (width 0.5) (layer "F.Cu") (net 19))
 (segment (start 89.535 61.595) (end 89.535 60.96) (width 0.5) (layer "F.Cu") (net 19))
 (segment (start 90.805 55.45) (end 90.805 60.325) (width 0.5) (layer "F.Cu") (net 18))
 (segment (start 93.98 63.5) (end 90.805 60.325) (width 0.5) (layer "F.Cu") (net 18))
 (segment (start 96.52 63.5) (end 92.075 59.055) (width 0.5) (layer "F.Cu") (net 17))
 (segment (start 92.075 59.055) (end 92.075 55.45) (width 0.5) (layer "F.Cu") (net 17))
 (segment (start 93.345 57.785) (end 93.345 55.45) (width 0.5) (layer "F.Cu") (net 16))
 (segment (start 99.06 63.5) (end 93.345 57.785) (width 0.5) (layer "F.Cu") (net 16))
 (segment (start 101.6 62.23) (end 101.6 63.5) (width 0.5) (layer "F.Cu") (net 15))
 (segment (start 99.695 60.325) (end 101.6 62.23) (width 0.5) (layer "F.Cu") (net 15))
 (segment (start 94.615 55.45) (end 94.615 57.15) (width 0.5) (layer "F.Cu") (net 15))
 (segment (start 97.79 60.325) (end 99.695 60.325) (width 0.5) (layer "F.Cu") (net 15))
 (segment (start 94.615 57.15) (end 97.79 60.325) (width 0.5) (layer "F.Cu") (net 15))
 (segment (start 97.79 59.055) (end 100.965 59.055) (width 0.5) (layer "F.Cu") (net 14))
 (segment (start 95.885 57.15) (end 97.79 59.055) (width 0.5) (layer "F.Cu") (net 14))
 (segment (start 100.965 59.055) (end 104.14 62.23) (width 0.5) (layer "F.Cu") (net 14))
 (segment (start 104.14 62.23) (end 104.14 63.5) (width 0.5) (layer "F.Cu") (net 14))
 (segment (start 95.885 55.45) (end 95.885 57.15) (width 0.5) (layer "F.Cu") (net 14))
 (segment (start 106.68 61.595) (end 102.87 57.785) (width 0.5) (layer "F.Cu") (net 13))
 (segment (start 102.87 57.785) (end 97.79 57.785) (width 0.5) (layer "F.Cu") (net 13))
 (segment (start 97.155 57.15) (end 97.155 55.45) (width 0.5) (layer "F.Cu") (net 13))
 (segment (start 106.68 63.5) (end 106.68 61.595) (width 0.5) (layer "F.Cu") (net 13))
 (segment (start 97.79 57.785) (end 97.155 57.15) (width 0.5) (layer "F.Cu") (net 13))
 (segment (start 113.03 55.245) (end 115.57 55.245) (width 0.5) (layer "F.Cu") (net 21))
 (segment (start 118.745 52.07) (end 118.745 50.165) (width 0.5) (layer "F.Cu") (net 21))
 (segment (start 118.745 50.165) (end 120.65 48.26) (width 0.5) (layer "F.Cu") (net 21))
 (segment (start 115.57 55.245) (end 118.745 52.07) (width 0.5) (layer "F.Cu") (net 21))
 (segment (start 113.03 53.275) (end 113.03 55.245) (width 0.5) (layer "F.Cu") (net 21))
 (segment (start 112.395 56.515) (end 118.11 56.515) (width 0.5) (layer "F.Cu") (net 23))
 (segment (start 119.38 63.5) (end 119.38 61.595) (width 0.5) (layer "F.Cu") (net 23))
 (segment (start 118.84 61.055) (end 118.84 59.785) (width 0.5) (layer "F.Cu") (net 23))
 (segment (start 111.76 55.88) (end 112.395 56.515) (width 0.5) (layer "F.Cu") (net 23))
 (segment (start 118.84 57.245) (end 118.84 58.42) (width 0.5) (layer "F.Cu") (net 23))
 (segment (start 111.76 53.275) (end 111.76 55.88) (width 0.5) (layer "F.Cu") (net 23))
 (segment (start 118.11 56.515) (end 118.84 57.245) (width 0.5) (layer "F.Cu") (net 23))
 (segment (start 119.38 61.595) (end 118.84 61.055) (width 0.5) (layer "F.Cu") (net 23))
 (segment (start 118.84 58.42) (end 118.84 59.785) (width 0.5) (layer "F.Cu") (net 23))
 (segment (start 100.965 45.085) (end 100.965 45.085) (width 0.5) (layer "F.Cu") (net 22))
 (segment (start 106.045 42.545) (end 106.045 42.545) (width 0.5) (layer "F.Cu") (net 22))
 (segment (start 114.3 42.545) (end 106.045 42.545) (width 0.5) (layer "F.Cu") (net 22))
 (segment (start 121.92 62.23) (end 123.5075 60.6425) (width 0.5) (layer "F.Cu") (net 22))
 (segment (start 99.9 46.15) (end 100.965 45.085) (width 0.5) (layer "F.Cu") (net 22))
 (segment (start 123.5075 58.42) (end 123.5075 60.6425) (width 0.5) (layer "F.Cu") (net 22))
 (segment (start 113.03 48.325) (end 114.3 48.325) (width 0.5) (layer "F.Cu") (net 22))
 (segment (start 98.425 46.15) (end 99.9 46.15) (width 0.5) (layer "F.Cu") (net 22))
 (segment (start 122.555 40.64) (end 117.475 40.64) (width 0.5) (layer "F.Cu") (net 22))
 (segment (start 113.03 48.325) (end 113.03 42.545) (width 0.5) (layer "F.Cu") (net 22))
 (segment (start 123.5075 58.42) (end 123.5075 41.5925) (width 0.5) (layer "F.Cu") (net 22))
 (segment (start 115.57 42.545) (end 114.3 42.545) (width 0.5) (layer "F.Cu") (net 22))
 (segment (start 123.46 58.4675) (end 123.5075 58.42) (width 0.5) (layer "F.Cu") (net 22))
 (segment (start 121.92 63.5) (end 121.92 62.23) (width 0.5) (layer "F.Cu") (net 22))
 (segment (start 117.475 40.64) (end 115.57 42.545) (width 0.5) (layer "F.Cu") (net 22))
 (segment (start 121.285 58.4675) (end 123.46 58.4675) (width 0.5) (layer "F.Cu") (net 22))
 (segment (start 123.5075 41.5925) (end 122.555 40.64) (width 0.5) (layer "F.Cu") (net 22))
 (via (at 106.045 42.545) (size 1.5) (drill 0.5) (layers "F.Cu" "B.Cu") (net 22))
 (via (at 100.965 45.085) (size 1.5) (drill 0.5) (layers "F.Cu" "B.Cu") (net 22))
 (segment (start 103.505 42.545) (end 100.965 45.085) (width 0.5) (layer "B.Cu") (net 22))
 (segment (start 106.045 42.545) (end 103.505 42.545) (width 0.5) (layer "B.Cu") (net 22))
 (segment (start 86.995 55.45) (end 86.995 64.77) (width 0.5) (layer "F.Cu") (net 24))
 (segment (start 111.76 64.77) (end 111.76 63.5) (width 0.5) (layer "F.Cu") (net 24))
 (segment (start 87.63 65.405) (end 111.125 65.405) (width 0.5) (layer "F.Cu") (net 24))
 (segment (start 86.995 64.77) (end 87.63 65.405) (width 0.5) (layer "F.Cu") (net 24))
 (segment (start 111.125 65.405) (end 111.76 64.77) (width 0.5) (layer "F.Cu") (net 24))
 (segment (start 110.49 48.325) (end 111.76 48.325) (width 0.5) (layer "F.Cu") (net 25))
 (segment (start 100.965 53.975) (end 100.965 53.975) (width 0.5) (layer "F.Cu") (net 26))
 (segment (start 97.155 46.15) (end 97.155 52.07) (width 0.5) (layer "F.Cu") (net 26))
 (segment (start 98.425 53.34) (end 100.33 53.34) (width 0.5) (layer "F.Cu") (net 26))
 (segment (start 104.84 53.275) (end 104.14 53.975) (width 0.5) (layer "F.Cu") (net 26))
 (segment (start 100.33 53.34) (end 100.965 53.975) (width 0.5) (layer "F.Cu") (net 26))
 (segment (start 97.155 52.07) (end 98.425 53.34) (width 0.5) (layer "F.Cu") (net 26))
 (segment (start 106.68 53.275) (end 104.84 53.275) (width 0.5) (layer "F.Cu") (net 26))
 (via (at 100.965 53.975) (size 1.5) (drill 0.5) (layers "F.Cu" "B.Cu") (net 26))
 (via (at 104.14 53.975) (size 1.5) (drill 0.5) (layers "F.Cu" "B.Cu") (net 26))
 (segment (start 100.965 53.975) (end 104.14 53.975) (width 0.5) (layer "B.Cu") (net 26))
 (segment (start 107.95 53.275) (end 110.49 53.275) (width 0.5) (layer "F.Cu") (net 27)))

